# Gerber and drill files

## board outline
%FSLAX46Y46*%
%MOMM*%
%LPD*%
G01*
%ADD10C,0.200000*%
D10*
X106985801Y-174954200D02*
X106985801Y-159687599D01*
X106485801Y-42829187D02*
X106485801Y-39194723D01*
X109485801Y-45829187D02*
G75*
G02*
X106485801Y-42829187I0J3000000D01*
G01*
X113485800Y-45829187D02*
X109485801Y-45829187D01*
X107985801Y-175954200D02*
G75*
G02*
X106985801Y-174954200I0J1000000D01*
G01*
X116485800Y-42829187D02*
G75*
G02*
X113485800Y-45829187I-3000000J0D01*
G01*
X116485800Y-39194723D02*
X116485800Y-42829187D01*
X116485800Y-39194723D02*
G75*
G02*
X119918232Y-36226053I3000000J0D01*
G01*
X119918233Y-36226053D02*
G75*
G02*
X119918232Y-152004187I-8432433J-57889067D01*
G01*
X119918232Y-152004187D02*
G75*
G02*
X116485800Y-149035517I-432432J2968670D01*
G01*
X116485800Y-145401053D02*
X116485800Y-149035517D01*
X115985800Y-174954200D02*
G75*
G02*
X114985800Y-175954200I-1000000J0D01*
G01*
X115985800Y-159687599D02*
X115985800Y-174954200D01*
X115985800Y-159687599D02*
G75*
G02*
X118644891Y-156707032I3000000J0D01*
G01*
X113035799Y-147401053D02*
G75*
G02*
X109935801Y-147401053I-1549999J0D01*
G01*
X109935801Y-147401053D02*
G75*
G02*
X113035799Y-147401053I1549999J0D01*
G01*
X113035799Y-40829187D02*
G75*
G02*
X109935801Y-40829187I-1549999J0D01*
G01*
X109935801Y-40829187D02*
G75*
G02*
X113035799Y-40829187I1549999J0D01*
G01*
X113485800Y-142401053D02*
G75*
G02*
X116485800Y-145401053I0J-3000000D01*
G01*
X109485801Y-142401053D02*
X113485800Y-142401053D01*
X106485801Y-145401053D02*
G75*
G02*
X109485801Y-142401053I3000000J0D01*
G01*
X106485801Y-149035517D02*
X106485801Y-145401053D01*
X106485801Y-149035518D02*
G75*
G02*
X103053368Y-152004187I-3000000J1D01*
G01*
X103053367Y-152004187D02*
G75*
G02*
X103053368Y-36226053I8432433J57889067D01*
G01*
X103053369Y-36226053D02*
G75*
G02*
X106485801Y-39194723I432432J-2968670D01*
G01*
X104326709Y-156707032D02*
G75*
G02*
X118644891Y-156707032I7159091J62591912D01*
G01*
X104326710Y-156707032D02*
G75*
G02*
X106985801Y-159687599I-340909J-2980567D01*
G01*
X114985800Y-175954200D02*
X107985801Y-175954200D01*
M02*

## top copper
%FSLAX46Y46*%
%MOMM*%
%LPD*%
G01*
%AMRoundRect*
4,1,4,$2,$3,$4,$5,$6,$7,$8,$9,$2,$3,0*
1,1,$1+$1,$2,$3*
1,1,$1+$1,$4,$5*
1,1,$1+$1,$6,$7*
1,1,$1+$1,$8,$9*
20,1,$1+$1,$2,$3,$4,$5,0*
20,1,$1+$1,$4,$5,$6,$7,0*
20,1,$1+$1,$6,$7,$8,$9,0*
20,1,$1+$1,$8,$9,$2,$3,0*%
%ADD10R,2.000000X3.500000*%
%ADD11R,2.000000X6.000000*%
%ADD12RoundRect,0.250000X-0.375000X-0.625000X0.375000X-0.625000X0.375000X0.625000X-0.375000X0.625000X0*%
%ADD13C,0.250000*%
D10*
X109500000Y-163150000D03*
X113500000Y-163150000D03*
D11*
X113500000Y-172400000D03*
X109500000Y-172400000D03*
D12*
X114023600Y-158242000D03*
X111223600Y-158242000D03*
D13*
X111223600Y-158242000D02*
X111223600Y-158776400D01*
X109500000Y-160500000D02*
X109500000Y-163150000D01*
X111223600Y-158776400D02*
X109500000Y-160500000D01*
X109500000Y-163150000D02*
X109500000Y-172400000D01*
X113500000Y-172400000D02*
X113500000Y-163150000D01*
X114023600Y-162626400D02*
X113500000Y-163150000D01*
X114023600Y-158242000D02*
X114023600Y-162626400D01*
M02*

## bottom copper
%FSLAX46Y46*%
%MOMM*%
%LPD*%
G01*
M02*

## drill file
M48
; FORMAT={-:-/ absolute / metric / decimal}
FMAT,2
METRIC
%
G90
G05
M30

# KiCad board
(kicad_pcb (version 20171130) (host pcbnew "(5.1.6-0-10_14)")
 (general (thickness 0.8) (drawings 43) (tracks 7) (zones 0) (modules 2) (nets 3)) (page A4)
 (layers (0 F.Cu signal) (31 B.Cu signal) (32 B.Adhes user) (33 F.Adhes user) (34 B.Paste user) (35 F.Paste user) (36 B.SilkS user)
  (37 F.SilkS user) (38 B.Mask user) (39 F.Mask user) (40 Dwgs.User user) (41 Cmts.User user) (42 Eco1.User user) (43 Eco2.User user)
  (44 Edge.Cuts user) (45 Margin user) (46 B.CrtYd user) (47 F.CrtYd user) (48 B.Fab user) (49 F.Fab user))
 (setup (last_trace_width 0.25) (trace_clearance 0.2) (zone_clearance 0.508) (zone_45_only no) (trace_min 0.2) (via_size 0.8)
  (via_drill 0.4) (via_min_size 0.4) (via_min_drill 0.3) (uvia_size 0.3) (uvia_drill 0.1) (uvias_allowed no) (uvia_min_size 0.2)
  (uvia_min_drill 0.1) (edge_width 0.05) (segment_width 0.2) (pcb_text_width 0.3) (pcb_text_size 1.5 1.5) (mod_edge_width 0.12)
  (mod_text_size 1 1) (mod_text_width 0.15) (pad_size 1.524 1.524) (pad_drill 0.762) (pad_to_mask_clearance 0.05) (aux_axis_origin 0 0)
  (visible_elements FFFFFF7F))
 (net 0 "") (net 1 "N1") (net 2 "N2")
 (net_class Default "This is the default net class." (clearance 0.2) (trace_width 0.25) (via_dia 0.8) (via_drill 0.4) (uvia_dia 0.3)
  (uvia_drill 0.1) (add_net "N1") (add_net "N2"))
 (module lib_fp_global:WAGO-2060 (layer F.Cu) (at 111.5 168.4 90)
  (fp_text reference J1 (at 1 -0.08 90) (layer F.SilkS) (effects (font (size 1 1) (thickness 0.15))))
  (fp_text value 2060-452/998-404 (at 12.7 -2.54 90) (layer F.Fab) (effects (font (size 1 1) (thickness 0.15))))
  (pad 1 smd rect (at 5.25 -2 90) (size 3.5 2) (layers F.Cu F.Paste F.Mask) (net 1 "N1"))
  (pad 2 smd rect (at 5.25 2 90) (size 3.5 2) (layers F.Cu F.Paste F.Mask) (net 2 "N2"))
  (pad 2 smd rect (at -4 2 90) (size 6 2) (layers F.Cu F.Paste F.Mask) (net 2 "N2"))
  (pad 1 smd rect (at -4 -2 90) (size 6 2) (layers F.Cu F.Paste F.Mask) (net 1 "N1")))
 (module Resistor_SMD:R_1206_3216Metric (layer F.Cu) (at 112.6236 158.242)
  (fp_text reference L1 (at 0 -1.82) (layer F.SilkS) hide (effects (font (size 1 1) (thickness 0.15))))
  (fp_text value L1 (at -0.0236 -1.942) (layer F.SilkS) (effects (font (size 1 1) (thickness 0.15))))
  (pad 2 smd roundrect (at 1.4 0) (size 1.25 1.75) (layers F.Cu F.Paste F.Mask) (roundrect_rratio 0.2) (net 2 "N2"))
  (pad 1 smd roundrect (at -1.4 0) (size 1.25 1.75) (layers F.Cu F.Paste F.Mask) (roundrect_rratio 0.2) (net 1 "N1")))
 (gr_line (start 106.985801 174.9542) (end 106.985801 159.687599) (layer Edge.Cuts) (width 0.2))
 (gr_line (start 106.485801 42.829187) (end 106.485801 39.194723) (layer Edge.Cuts) (width 0.2))
 (gr_arc (start 109.485801 42.829187) (end 106.485801 42.829187) (angle -90) (layer Edge.Cuts) (width 0.2))
 (gr_line (start 113.4858 45.829187) (end 109.485801 45.829187) (layer Edge.Cuts) (width 0.2))
 (gr_arc (start 107.985801 174.9542) (end 106.985801 174.9542) (angle -90) (layer Edge.Cuts) (width 0.2))
 (gr_arc (start 113.4858 42.829187) (end 113.4858 45.829187) (angle -90) (layer Edge.Cuts) (width 0.2))
 (gr_line (start 116.4858 39.194723) (end 116.4858 42.829187) (layer Edge.Cuts) (width 0.2))
 (gr_arc (start 119.4858 39.194723) (end 119.918232 36.226053) (angle -98.28772162) (layer Edge.Cuts) (width 0.2))
 (gr_arc (start 111.4858 94.11512) (end 119.918232 152.004187) (angle -163.4245568) (layer Edge.Cuts) (width 0.2))
 (gr_arc (start 119.4858 149.035517) (end 116.4858 149.035517) (angle -98.28772162) (layer Edge.Cuts) (width 0.2))
 (gr_line (start 116.4858 145.401053) (end 116.4858 149.035517) (layer Edge.Cuts) (width 0.2))
 (gr_arc (start 114.9858 174.9542) (end 114.9858 175.9542) (angle -90) (layer Edge.Cuts) (width 0.2))
 (gr_line (start 115.9858 159.687599) (end 115.9858 174.9542) (layer Edge.Cuts) (width 0.2))
 (gr_arc (start 118.9858 159.687599) (end 118.644891 156.707032) (angle -83.47502116) (layer Edge.Cuts) (width 0.2))
 (gr_circle (center 111.4858 147.401053) (end 109.935801 147.401053) (layer Edge.Cuts) (width 0.2))
 (gr_circle (center 111.4858 40.829187) (end 109.935801 40.829187) (layer Edge.Cuts) (width 0.2))
 (gr_arc (start 113.4858 145.401053) (end 116.4858 145.401053) (angle -90) (layer Edge.Cuts) (width 0.2))
 (gr_line (start 109.485801 142.401053) (end 113.4858 142.401053) (layer Edge.Cuts) (width 0.2))
 (gr_arc (start 109.485801 145.401053) (end 109.485801 142.401053) (angle -90) (layer Edge.Cuts) (width 0.2))
 (gr_line (start 106.485801 149.035517) (end 106.485801 145.401053) (layer Edge.Cuts) (width 0.2))
 (gr_arc (start 103.485801 149.035517) (end 103.053368 152.004187) (angle -98.28772162) (layer Edge.Cuts) (width 0.2))
 (gr_arc (start 111.4858 94.11512) (end 103.053368 36.226053) (angle -163.4245568) (layer Edge.Cuts) (width 0.2))
 (gr_arc (start 103.485801 39.194723) (end 106.485801 39.194723) (angle -98.28772162) (layer Edge.Cuts) (width 0.2))
 (gr_arc (start 111.4858 94.11512) (end 118.644891 156.707032) (angle -346.9500423) (layer Edge.Cuts) (width 0.2))
 (gr_arc (start 103.985801 159.687599) (end 106.985801 159.687599) (angle -83.47502116) (layer Edge.Cuts) (width 0.2))
 (gr_line (start 114.9858 175.9542) (end 107.985801 175.9542) (layer Edge.Cuts) (width 0.2))
 (segment (start 111.2236 158.242) (end 111.2236 158.7764) (width 0.25) (layer F.Cu) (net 1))
 (segment (start 109.5 160.5) (end 109.5 163.15) (width 0.25) (layer F.Cu) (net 1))
 (segment (start 111.2236 158.7764) (end 109.5 160.5) (width 0.25) (layer F.Cu) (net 1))
 (segment (start 109.5 163.15) (end 109.5 172.4) (width 0.25) (layer F.Cu) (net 1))
 (segment (start 113.5 172.4) (end 113.5 163.15) (width 0.25) (layer F.Cu) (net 2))
 (segment (start 114.0236 162.6264) (end 113.5 163.15) (width 0.25) (layer F.Cu) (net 2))
 (segment (start 114.0236 158.242) (end 114.0236 162.6264) (width 0.25) (layer F.Cu) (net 2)))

